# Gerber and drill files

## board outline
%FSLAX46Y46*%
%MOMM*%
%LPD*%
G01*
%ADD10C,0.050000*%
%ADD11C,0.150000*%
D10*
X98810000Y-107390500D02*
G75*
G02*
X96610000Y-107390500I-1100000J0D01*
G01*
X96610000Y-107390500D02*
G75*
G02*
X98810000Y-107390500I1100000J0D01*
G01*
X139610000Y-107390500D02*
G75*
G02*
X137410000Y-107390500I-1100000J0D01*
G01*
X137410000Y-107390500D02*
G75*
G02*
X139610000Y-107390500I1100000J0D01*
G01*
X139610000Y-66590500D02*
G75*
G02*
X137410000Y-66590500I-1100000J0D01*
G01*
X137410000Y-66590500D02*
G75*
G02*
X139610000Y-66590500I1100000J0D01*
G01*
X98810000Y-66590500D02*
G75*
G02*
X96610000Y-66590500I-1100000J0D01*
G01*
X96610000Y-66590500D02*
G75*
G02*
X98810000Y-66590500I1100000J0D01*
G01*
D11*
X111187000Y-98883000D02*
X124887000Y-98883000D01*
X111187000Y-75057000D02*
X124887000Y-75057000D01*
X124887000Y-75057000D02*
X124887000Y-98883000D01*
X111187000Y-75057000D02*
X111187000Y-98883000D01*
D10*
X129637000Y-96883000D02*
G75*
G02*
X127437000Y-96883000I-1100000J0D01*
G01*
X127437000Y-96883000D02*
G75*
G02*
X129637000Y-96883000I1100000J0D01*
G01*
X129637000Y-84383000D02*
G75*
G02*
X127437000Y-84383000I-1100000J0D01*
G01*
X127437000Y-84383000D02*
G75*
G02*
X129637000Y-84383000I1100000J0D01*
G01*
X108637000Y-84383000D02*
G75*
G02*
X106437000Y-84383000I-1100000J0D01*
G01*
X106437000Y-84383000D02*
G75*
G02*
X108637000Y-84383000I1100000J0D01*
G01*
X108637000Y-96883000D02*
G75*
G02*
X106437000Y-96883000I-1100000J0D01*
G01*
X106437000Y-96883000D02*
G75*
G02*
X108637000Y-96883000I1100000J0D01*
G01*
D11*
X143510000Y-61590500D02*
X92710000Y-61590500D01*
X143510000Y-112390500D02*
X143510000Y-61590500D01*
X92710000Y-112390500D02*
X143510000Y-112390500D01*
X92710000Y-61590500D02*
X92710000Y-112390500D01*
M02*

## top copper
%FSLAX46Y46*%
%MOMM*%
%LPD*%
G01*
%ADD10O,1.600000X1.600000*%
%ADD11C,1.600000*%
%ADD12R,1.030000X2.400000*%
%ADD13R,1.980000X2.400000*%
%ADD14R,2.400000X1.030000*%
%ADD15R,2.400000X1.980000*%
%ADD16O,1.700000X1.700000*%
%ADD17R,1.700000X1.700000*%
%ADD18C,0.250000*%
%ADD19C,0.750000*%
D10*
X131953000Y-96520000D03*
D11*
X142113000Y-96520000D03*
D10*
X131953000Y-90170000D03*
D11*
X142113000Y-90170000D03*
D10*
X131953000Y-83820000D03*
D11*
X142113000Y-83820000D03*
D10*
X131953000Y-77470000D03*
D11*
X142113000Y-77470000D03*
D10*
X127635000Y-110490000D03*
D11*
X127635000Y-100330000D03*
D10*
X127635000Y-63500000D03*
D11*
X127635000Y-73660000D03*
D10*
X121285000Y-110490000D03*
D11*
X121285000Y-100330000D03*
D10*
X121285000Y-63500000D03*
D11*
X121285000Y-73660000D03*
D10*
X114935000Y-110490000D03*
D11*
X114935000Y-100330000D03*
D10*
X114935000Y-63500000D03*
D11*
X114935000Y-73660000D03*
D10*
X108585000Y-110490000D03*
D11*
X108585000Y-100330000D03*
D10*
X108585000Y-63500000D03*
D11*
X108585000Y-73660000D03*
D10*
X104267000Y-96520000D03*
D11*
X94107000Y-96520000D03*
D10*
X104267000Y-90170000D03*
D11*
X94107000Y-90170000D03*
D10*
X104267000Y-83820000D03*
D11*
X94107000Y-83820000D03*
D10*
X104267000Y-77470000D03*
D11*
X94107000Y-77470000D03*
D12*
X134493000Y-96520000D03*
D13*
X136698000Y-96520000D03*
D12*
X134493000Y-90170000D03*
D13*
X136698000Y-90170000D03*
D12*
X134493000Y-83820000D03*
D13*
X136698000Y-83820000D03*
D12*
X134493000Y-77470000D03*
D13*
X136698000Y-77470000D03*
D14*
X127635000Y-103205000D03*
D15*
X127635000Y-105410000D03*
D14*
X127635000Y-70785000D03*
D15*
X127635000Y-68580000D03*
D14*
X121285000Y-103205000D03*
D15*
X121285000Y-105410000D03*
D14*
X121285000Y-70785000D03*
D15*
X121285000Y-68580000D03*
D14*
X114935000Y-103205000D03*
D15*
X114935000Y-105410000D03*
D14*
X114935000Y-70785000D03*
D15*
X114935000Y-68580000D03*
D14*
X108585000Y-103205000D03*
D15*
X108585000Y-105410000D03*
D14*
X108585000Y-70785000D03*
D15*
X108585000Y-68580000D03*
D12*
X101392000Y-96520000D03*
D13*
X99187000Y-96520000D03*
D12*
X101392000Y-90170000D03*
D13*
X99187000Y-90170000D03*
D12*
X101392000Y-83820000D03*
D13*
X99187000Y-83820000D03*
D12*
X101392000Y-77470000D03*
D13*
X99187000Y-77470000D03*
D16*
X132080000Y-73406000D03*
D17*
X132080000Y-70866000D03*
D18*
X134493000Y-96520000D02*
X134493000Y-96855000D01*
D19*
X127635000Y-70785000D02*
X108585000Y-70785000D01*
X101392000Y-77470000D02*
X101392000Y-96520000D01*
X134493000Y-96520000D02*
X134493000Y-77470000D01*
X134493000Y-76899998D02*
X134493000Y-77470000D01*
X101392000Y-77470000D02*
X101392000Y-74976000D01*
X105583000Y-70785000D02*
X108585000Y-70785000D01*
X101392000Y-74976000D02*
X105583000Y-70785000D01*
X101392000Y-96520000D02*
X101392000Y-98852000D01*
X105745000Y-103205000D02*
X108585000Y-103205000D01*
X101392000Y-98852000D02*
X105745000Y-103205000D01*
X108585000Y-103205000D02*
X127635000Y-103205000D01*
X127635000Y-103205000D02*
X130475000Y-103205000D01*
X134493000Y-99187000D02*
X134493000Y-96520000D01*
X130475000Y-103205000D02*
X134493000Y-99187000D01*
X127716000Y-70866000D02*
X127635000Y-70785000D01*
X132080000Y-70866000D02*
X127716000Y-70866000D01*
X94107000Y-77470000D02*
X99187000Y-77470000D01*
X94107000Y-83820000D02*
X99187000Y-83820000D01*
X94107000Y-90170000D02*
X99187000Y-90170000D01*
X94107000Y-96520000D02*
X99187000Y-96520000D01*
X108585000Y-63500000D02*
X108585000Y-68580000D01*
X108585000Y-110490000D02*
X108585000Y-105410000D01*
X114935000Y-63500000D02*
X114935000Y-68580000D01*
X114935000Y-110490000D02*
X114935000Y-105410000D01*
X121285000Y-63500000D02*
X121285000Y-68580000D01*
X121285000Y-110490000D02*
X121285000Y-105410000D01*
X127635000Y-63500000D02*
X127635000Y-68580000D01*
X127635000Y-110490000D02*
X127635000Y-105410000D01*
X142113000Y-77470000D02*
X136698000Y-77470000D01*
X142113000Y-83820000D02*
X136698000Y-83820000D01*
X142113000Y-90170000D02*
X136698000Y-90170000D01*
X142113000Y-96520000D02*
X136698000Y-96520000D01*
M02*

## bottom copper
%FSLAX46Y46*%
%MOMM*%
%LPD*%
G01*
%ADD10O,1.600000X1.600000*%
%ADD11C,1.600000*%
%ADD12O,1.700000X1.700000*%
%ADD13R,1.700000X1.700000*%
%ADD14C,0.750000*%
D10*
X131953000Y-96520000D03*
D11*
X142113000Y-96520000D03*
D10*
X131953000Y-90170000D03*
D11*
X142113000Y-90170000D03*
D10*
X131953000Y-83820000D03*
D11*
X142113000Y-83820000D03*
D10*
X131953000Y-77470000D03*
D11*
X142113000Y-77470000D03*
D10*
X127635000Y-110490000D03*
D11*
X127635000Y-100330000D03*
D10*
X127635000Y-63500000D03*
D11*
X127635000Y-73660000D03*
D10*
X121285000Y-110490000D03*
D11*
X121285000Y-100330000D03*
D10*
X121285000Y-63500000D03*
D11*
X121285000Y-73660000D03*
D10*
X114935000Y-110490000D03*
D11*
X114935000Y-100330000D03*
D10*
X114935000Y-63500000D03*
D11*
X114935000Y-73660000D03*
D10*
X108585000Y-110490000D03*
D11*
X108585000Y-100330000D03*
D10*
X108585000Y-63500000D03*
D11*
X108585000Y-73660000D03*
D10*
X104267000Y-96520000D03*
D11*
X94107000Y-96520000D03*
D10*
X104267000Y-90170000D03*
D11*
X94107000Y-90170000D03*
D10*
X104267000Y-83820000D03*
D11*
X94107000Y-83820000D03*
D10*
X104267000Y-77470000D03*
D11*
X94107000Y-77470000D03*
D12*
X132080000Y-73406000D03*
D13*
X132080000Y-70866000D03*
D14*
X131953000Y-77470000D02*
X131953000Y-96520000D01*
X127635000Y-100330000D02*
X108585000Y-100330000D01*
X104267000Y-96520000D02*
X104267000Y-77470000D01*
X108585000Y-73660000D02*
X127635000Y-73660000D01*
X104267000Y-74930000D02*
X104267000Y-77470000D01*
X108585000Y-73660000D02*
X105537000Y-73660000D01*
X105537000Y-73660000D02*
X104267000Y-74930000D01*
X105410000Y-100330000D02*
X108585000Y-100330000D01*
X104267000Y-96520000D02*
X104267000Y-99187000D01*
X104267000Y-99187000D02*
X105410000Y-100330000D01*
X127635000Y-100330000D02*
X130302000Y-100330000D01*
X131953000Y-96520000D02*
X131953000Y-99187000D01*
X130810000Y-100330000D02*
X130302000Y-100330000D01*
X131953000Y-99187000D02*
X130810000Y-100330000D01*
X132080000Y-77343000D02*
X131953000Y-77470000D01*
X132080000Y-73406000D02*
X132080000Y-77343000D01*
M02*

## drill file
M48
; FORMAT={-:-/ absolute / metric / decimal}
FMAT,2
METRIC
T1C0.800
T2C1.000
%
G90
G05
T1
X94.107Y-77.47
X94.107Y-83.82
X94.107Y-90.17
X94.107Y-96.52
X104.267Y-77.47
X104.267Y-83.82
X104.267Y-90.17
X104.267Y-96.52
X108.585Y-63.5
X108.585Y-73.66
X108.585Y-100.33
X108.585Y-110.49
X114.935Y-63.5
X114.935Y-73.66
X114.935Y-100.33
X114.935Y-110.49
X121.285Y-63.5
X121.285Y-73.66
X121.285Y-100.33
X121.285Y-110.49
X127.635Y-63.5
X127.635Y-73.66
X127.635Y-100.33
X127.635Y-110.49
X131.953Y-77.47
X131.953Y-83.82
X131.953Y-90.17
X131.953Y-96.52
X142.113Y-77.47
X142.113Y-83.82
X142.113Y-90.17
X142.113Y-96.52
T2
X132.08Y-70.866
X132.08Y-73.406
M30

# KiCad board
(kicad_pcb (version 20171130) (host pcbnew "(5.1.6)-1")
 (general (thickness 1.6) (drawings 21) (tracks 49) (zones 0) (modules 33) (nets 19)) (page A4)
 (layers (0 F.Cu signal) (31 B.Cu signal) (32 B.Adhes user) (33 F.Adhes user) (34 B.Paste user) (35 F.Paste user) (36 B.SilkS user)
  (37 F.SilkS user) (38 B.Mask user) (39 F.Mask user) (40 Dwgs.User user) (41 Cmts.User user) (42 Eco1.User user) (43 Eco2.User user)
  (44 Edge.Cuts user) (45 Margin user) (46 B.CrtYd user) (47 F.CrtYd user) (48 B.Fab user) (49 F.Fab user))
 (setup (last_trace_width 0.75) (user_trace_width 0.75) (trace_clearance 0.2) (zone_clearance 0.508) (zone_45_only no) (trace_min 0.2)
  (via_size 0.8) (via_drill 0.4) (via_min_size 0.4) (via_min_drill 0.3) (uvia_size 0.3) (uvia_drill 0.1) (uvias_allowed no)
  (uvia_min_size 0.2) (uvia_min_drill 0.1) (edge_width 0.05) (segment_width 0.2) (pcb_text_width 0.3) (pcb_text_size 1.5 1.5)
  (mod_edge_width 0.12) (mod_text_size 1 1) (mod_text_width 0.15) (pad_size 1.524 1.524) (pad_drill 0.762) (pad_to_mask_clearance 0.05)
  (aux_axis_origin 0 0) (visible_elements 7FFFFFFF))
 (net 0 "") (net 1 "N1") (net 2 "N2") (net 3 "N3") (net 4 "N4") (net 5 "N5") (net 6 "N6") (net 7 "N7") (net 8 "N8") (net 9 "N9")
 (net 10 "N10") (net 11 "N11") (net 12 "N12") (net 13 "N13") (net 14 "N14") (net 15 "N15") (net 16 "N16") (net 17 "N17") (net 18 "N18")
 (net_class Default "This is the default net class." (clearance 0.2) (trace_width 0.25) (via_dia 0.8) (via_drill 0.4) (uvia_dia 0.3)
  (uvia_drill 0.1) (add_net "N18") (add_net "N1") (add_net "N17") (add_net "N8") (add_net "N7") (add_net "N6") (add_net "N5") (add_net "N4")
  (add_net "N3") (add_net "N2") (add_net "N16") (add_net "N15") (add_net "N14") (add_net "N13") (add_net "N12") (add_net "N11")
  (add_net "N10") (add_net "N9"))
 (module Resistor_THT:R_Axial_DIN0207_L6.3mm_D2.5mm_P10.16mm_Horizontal (layer B.Cu) (at 142.113 96.52 180)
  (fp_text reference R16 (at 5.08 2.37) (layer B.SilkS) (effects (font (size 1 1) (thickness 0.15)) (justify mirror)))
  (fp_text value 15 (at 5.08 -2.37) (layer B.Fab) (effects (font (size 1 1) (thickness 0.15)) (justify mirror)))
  (pad 2 thru_hole oval (at 10.16 0 180) (size 1.6 1.6) (drill 0.8) (layers *.Cu *.Mask) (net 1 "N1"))
  (pad 1 thru_hole circle (at 0 0 180) (size 1.6 1.6) (drill 0.8) (layers *.Cu *.Mask) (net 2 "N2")))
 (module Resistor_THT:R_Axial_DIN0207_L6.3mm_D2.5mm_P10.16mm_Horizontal (layer B.Cu) (at 142.113 90.17 180)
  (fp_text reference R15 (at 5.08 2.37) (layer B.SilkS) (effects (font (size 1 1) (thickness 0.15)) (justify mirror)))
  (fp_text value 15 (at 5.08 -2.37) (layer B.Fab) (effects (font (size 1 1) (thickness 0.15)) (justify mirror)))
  (pad 2 thru_hole oval (at 10.16 0 180) (size 1.6 1.6) (drill 0.8) (layers *.Cu *.Mask) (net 1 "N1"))
  (pad 1 thru_hole circle (at 0 0 180) (size 1.6 1.6) (drill 0.8) (layers *.Cu *.Mask) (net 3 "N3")))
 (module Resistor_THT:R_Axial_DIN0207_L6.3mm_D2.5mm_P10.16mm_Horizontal (layer B.Cu) (at 142.113 83.82 180)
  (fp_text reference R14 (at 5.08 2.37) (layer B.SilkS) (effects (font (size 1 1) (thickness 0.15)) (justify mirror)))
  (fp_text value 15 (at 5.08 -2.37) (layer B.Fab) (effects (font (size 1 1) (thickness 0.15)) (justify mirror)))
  (pad 2 thru_hole oval (at 10.16 0 180) (size 1.6 1.6) (drill 0.8) (layers *.Cu *.Mask) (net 1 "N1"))
  (pad 1 thru_hole circle (at 0 0 180) (size 1.6 1.6) (drill 0.8) (layers *.Cu *.Mask) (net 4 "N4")))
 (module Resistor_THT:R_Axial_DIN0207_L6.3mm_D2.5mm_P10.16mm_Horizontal (layer B.Cu) (at 142.113 77.47 180)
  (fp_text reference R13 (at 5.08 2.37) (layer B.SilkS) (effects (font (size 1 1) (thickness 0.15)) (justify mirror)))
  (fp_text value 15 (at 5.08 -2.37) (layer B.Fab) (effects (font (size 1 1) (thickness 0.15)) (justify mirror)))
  (pad 2 thru_hole oval (at 10.16 0 180) (size 1.6 1.6) (drill 0.8) (layers *.Cu *.Mask) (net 1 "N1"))
  (pad 1 thru_hole circle (at 0 0 180) (size 1.6 1.6) (drill 0.8) (layers *.Cu *.Mask) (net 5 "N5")))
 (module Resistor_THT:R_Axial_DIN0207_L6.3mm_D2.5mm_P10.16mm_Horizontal (layer B.Cu) (at 127.635 100.33 270)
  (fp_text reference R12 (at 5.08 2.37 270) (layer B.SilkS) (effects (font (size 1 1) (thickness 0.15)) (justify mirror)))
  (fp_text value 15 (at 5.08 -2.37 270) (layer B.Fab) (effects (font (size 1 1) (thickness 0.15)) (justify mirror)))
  (pad 2 thru_hole oval (at 10.16 0 270) (size 1.6 1.6) (drill 0.8) (layers *.Cu *.Mask) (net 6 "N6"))
  (pad 1 thru_hole circle (at 0 0 270) (size 1.6 1.6) (drill 0.8) (layers *.Cu *.Mask) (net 1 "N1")))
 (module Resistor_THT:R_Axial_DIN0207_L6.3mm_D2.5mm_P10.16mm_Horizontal (layer B.Cu) (at 127.635 73.66 90)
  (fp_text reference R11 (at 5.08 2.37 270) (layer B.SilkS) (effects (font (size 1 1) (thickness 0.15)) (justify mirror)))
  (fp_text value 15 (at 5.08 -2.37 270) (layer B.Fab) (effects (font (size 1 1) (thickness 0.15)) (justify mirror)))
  (pad 2 thru_hole oval (at 10.16 0 90) (size 1.6 1.6) (drill 0.8) (layers *.Cu *.Mask) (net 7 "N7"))
  (pad 1 thru_hole circle (at 0 0 90) (size 1.6 1.6) (drill 0.8) (layers *.Cu *.Mask) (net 1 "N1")))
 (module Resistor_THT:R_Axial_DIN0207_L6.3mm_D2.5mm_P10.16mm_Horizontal (layer B.Cu) (at 121.285 100.33 270)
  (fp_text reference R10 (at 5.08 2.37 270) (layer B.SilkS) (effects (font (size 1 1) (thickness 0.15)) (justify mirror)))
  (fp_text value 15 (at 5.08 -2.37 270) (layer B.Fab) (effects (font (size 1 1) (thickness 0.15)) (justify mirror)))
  (pad 2 thru_hole oval (at 10.16 0 270) (size 1.6 1.6) (drill 0.8) (layers *.Cu *.Mask) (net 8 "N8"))
  (pad 1 thru_hole circle (at 0 0 270) (size 1.6 1.6) (drill 0.8) (layers *.Cu *.Mask) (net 1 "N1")))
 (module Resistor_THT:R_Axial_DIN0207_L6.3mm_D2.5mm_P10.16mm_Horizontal (layer B.Cu) (at 121.285 73.66 90)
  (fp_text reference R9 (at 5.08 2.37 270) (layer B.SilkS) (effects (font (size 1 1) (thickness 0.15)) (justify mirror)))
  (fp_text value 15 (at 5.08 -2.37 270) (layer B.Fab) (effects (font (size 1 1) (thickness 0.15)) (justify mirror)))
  (pad 2 thru_hole oval (at 10.16 0 90) (size 1.6 1.6) (drill 0.8) (layers *.Cu *.Mask) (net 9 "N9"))
  (pad 1 thru_hole circle (at 0 0 90) (size 1.6 1.6) (drill 0.8) (layers *.Cu *.Mask) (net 1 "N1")))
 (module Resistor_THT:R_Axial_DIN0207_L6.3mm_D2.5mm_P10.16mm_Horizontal (layer B.Cu) (at 114.935 100.33 270)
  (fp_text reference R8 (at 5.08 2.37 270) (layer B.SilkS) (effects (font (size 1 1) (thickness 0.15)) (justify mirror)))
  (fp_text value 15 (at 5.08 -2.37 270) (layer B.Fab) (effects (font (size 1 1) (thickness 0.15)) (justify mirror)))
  (pad 2 thru_hole oval (at 10.16 0 270) (size 1.6 1.6) (drill 0.8) (layers *.Cu *.Mask) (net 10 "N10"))
  (pad 1 thru_hole circle (at 0 0 270) (size 1.6 1.6) (drill 0.8) (layers *.Cu *.Mask) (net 1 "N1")))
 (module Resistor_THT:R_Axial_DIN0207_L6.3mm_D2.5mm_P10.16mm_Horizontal (layer B.Cu) (at 114.935 73.66 90)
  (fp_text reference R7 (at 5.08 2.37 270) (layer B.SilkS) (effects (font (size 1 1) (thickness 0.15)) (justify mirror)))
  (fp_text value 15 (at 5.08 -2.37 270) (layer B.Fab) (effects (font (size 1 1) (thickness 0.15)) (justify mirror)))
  (pad 2 thru_hole oval (at 10.16 0 90) (size 1.6 1.6) (drill 0.8) (layers *.Cu *.Mask) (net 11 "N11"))
  (pad 1 thru_hole circle (at 0 0 90) (size 1.6 1.6) (drill 0.8) (layers *.Cu *.Mask) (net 1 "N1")))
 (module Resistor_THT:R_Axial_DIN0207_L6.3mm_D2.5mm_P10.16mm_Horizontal (layer B.Cu) (at 108.585 100.33 270)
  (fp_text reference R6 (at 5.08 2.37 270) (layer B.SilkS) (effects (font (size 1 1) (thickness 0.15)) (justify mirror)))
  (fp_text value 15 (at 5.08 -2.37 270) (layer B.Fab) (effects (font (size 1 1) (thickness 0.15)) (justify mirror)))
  (pad 2 thru_hole oval (at 10.16 0 270) (size 1.6 1.6) (drill 0.8) (layers *.Cu *.Mask) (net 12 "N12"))
  (pad 1 thru_hole circle (at 0 0 270) (size 1.6 1.6) (drill 0.8) (layers *.Cu *.Mask) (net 1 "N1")))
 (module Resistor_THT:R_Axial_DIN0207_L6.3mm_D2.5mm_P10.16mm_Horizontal (layer B.Cu) (at 108.585 73.66 90)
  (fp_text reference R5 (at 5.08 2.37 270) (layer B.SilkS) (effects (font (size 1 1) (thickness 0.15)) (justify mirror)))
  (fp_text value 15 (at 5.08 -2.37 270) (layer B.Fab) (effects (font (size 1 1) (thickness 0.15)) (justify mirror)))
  (pad 2 thru_hole oval (at 10.16 0 90) (size 1.6 1.6) (drill 0.8) (layers *.Cu *.Mask) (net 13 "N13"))
  (pad 1 thru_hole circle (at 0 0 90) (size 1.6 1.6) (drill 0.8) (layers *.Cu *.Mask) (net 1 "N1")))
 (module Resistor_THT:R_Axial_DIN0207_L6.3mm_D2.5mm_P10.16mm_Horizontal (layer B.Cu) (at 94.107 96.52)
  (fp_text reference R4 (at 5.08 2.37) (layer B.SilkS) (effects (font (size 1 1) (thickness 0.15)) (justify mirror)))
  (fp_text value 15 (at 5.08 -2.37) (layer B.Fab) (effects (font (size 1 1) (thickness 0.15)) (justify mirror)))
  (pad 2 thru_hole oval (at 10.16 0) (size 1.6 1.6) (drill 0.8) (layers *.Cu *.Mask) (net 1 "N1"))
  (pad 1 thru_hole circle (at 0 0) (size 1.6 1.6) (drill 0.8) (layers *.Cu *.Mask) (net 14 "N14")))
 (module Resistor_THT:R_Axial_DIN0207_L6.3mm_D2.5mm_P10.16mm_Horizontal (layer B.Cu) (at 94.107 90.17)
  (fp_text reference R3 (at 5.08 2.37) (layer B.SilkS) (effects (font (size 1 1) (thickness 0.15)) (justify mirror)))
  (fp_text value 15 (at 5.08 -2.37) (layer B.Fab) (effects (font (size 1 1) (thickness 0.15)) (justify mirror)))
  (pad 2 thru_hole oval (at 10.16 0) (size 1.6 1.6) (drill 0.8) (layers *.Cu *.Mask) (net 1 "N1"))
  (pad 1 thru_hole circle (at 0 0) (size 1.6 1.6) (drill 0.8) (layers *.Cu *.Mask) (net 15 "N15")))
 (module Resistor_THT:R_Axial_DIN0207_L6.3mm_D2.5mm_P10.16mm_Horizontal (layer B.Cu) (at 94.107 83.82)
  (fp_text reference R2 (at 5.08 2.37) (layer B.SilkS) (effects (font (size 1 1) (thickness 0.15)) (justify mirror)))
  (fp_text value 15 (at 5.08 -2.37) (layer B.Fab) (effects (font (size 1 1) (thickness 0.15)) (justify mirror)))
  (pad 2 thru_hole oval (at 10.16 0) (size 1.6 1.6) (drill 0.8) (layers *.Cu *.Mask) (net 1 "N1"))
  (pad 1 thru_hole circle (at 0 0) (size 1.6 1.6) (drill 0.8) (layers *.Cu *.Mask) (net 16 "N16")))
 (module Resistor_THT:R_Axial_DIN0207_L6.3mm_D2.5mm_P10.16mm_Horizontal (layer B.Cu) (at 94.107 77.47)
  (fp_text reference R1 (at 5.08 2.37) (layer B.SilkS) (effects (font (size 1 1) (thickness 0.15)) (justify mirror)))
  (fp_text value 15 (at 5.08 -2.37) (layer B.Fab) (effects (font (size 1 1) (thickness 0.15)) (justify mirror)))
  (pad 2 thru_hole oval (at 10.16 0) (size 1.6 1.6) (drill 0.8) (layers *.Cu *.Mask) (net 1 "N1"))
  (pad 1 thru_hole circle (at 0 0) (size 1.6 1.6) (drill 0.8) (layers *.Cu *.Mask) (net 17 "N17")))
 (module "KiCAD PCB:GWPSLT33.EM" (layer F.Cu) (at 135.838 96.52 180)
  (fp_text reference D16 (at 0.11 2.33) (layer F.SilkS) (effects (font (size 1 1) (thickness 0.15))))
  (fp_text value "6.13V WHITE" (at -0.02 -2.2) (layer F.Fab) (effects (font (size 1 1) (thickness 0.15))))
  (pad 2 smd rect (at 1.345 0 180) (size 1.03 2.4) (layers F.Cu F.Paste F.Mask) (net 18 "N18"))
  (pad 1 smd rect (at -0.86 0 180) (size 1.98 2.4) (layers F.Cu F.Paste F.Mask) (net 2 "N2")))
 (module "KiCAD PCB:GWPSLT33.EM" (layer F.Cu) (at 135.838 90.17 180)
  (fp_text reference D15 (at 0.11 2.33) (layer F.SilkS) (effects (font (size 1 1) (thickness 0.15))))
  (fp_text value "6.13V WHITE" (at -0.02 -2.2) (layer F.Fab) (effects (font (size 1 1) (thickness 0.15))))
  (pad 2 smd rect (at 1.345 0 180) (size 1.03 2.4) (layers F.Cu F.Paste F.Mask) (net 18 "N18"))
  (pad 1 smd rect (at -0.86 0 180) (size 1.98 2.4) (layers F.Cu F.Paste F.Mask) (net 3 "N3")))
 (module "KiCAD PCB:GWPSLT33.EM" (layer F.Cu) (at 135.838 83.82 180)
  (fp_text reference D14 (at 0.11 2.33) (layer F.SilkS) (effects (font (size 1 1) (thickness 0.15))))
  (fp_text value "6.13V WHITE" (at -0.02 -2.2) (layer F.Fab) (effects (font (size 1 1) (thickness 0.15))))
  (pad 2 smd rect (at 1.345 0 180) (size 1.03 2.4) (layers F.Cu F.Paste F.Mask) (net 18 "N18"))
  (pad 1 smd rect (at -0.86 0 180) (size 1.98 2.4) (layers F.Cu F.Paste F.Mask) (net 4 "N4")))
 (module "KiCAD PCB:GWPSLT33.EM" (layer F.Cu) (at 135.838 77.47 180)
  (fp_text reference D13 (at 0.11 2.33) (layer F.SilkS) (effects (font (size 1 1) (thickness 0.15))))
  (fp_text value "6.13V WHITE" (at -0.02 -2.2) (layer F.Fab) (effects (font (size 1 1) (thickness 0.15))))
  (pad 2 smd rect (at 1.345 0 180) (size 1.03 2.4) (layers F.Cu F.Paste F.Mask) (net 18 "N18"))
  (pad 1 smd rect (at -0.86 0 180) (size 1.98 2.4) (layers F.Cu F.Paste F.Mask) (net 5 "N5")))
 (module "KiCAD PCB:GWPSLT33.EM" (layer F.Cu) (at 127.635 104.55 90)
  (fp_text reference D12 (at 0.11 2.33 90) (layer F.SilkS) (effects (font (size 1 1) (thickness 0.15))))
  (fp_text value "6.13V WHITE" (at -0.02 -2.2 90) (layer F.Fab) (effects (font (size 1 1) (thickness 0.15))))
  (pad 2 smd rect (at 1.345 0 90) (size 1.03 2.4) (layers F.Cu F.Paste F.Mask) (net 18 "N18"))
  (pad 1 smd rect (at -0.86 0 90) (size 1.98 2.4) (layers F.Cu F.Paste F.Mask) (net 6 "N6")))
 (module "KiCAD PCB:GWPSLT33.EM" (layer F.Cu) (at 127.635 69.44 270)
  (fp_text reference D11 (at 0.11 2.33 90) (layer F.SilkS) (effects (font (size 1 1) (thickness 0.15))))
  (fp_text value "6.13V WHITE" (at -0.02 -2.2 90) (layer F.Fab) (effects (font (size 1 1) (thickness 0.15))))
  (pad 2 smd rect (at 1.345 0 270) (size 1.03 2.4) (layers F.Cu F.Paste F.Mask) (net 18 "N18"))
  (pad 1 smd rect (at -0.86 0 270) (size 1.98 2.4) (layers F.Cu F.Paste F.Mask) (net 7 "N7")))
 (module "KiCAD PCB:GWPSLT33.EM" (layer F.Cu) (at 121.285 104.55 90)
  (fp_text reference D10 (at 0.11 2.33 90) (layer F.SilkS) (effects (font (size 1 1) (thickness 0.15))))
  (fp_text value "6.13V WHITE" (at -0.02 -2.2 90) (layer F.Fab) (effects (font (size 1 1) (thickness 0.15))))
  (pad 2 smd rect (at 1.345 0 90) (size 1.03 2.4) (layers F.Cu F.Paste F.Mask) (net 18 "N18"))
  (pad 1 smd rect (at -0.86 0 90) (size 1.98 2.4) (layers F.Cu F.Paste F.Mask) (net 8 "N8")))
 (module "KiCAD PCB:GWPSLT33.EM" (layer F.Cu) (at 121.285 69.44 270)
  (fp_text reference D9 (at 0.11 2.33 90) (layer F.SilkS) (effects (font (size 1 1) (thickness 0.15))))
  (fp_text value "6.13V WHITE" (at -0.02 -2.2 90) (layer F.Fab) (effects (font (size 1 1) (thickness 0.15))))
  (pad 2 smd rect (at 1.345 0 270) (size 1.03 2.4) (layers F.Cu F.Paste F.Mask) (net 18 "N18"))
  (pad 1 smd rect (at -0.86 0 270) (size 1.98 2.4) (layers F.Cu F.Paste F.Mask) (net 9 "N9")))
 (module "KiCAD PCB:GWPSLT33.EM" (layer F.Cu) (at 114.935 104.55 90)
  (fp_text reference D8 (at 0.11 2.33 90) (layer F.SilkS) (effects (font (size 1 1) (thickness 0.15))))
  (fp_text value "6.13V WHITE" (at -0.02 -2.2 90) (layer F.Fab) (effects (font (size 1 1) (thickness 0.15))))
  (pad 2 smd rect (at 1.345 0 90) (size 1.03 2.4) (layers F.Cu F.Paste F.Mask) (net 18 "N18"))
  (pad 1 smd rect (at -0.86 0 90) (size 1.98 2.4) (layers F.Cu F.Paste F.Mask) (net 10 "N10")))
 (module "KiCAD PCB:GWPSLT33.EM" (layer F.Cu) (at 114.935 69.44 270)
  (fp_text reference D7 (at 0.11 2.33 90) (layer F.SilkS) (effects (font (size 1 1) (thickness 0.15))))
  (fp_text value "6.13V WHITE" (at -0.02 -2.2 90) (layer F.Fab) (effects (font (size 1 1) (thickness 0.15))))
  (pad 2 smd rect (at 1.345 0 270) (size 1.03 2.4) (layers F.Cu F.Paste F.Mask) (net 18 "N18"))
  (pad 1 smd rect (at -0.86 0 270) (size 1.98 2.4) (layers F.Cu F.Paste F.Mask) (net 11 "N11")))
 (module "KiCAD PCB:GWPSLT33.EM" (layer F.Cu) (at 108.585 104.55 90)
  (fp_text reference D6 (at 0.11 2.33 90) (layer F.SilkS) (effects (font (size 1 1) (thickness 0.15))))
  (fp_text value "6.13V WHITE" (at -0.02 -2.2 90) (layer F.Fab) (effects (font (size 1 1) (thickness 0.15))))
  (pad 2 smd rect (at 1.345 0 90) (size 1.03 2.4) (layers F.Cu F.Paste F.Mask) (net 18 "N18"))
  (pad 1 smd rect (at -0.86 0 90) (size 1.98 2.4) (layers F.Cu F.Paste F.Mask) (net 12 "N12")))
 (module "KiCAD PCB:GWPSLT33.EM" (layer F.Cu) (at 108.585 69.44 270)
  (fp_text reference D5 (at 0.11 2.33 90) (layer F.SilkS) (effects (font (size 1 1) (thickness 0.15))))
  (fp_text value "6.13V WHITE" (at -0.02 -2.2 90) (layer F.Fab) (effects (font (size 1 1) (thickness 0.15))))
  (pad 2 smd rect (at 1.345 0 270) (size 1.03 2.4) (layers F.Cu F.Paste F.Mask) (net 18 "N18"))
  (pad 1 smd rect (at -0.86 0 270) (size 1.98 2.4) (layers F.Cu F.Paste F.Mask) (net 13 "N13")))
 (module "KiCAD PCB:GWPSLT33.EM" (layer F.Cu) (at 100.047 96.52)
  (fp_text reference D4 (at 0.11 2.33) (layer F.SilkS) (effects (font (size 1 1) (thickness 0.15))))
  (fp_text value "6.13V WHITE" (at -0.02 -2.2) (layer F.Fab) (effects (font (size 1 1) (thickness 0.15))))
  (pad 2 smd rect (at 1.345 0) (size 1.03 2.4) (layers F.Cu F.Paste F.Mask) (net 18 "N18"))
  (pad 1 smd rect (at -0.86 0) (size 1.98 2.4) (layers F.Cu F.Paste F.Mask) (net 14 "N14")))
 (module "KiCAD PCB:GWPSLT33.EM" (layer F.Cu) (at 100.047 90.17)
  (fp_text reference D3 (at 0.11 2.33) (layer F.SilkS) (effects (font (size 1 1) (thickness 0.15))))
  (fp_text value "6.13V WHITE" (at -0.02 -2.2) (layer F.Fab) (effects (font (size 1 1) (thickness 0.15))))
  (pad 2 smd rect (at 1.345 0) (size 1.03 2.4) (layers F.Cu F.Paste F.Mask) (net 18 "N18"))
  (pad 1 smd rect (at -0.86 0) (size 1.98 2.4) (layers F.Cu F.Paste F.Mask) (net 15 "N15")))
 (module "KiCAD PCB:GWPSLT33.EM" (layer F.Cu) (at 100.047 83.82)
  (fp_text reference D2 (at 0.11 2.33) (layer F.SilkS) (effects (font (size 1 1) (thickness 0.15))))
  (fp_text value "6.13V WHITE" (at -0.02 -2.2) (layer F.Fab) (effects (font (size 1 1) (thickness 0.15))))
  (pad 2 smd rect (at 1.345 0) (size 1.03 2.4) (layers F.Cu F.Paste F.Mask) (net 18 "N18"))
  (pad 1 smd rect (at -0.86 0) (size 1.98 2.4) (layers F.Cu F.Paste F.Mask) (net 16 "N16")))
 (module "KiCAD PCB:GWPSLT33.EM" (layer F.Cu) (at 100.047 77.47)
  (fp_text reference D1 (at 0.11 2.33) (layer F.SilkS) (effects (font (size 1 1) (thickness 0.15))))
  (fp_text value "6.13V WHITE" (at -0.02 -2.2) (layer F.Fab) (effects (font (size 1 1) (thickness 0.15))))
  (pad 2 smd rect (at 1.345 0) (size 1.03 2.4) (layers F.Cu F.Paste F.Mask) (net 18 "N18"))
  (pad 1 smd rect (at -0.86 0) (size 1.98 2.4) (layers F.Cu F.Paste F.Mask) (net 17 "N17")))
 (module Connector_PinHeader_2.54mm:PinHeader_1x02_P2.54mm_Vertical (layer F.Cu) (at 132.08 70.866)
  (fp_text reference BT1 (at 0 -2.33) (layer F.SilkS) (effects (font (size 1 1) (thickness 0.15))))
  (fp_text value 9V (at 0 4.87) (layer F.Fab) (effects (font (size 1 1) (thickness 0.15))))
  (pad 2 thru_hole oval (at 0 2.54) (size 1.7 1.7) (drill 1) (layers *.Cu *.Mask) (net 1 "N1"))
  (pad 1 thru_hole rect (at 0 0) (size 1.7 1.7) (drill 1) (layers *.Cu *.Mask) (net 18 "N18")))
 (gr_circle (center 97.71 107.3905) (end 98.81 107.3905) (layer Edge.Cuts) (width 0.05))
 (gr_circle (center 138.51 107.3905) (end 139.61 107.3905) (layer Edge.Cuts) (width 0.05))
 (gr_circle (center 138.51 66.5905) (end 139.61 66.5905) (layer Edge.Cuts) (width 0.05))
 (gr_circle (center 97.71 66.5905) (end 98.81 66.5905) (layer Edge.Cuts) (width 0.05))
 (gr_line (start 111.187 98.883) (end 124.887 98.883) (layer Edge.Cuts) (width 0.15))
 (gr_line (start 111.187 75.057) (end 124.887 75.057) (layer Edge.Cuts) (width 0.15))
 (gr_line (start 124.887 75.057) (end 124.887 98.883) (layer Edge.Cuts) (width 0.15))
 (gr_line (start 111.187 75.057) (end 111.187 98.883) (layer Edge.Cuts) (width 0.15))
 (gr_circle (center 128.537 96.883) (end 129.637 96.883) (layer Edge.Cuts) (width 0.05))
 (gr_circle (center 128.537 84.383) (end 129.637 84.383) (layer Edge.Cuts) (width 0.05))
 (gr_circle (center 107.537 84.383) (end 108.637 84.383) (layer Edge.Cuts) (width 0.05))
 (gr_circle (center 107.537 96.883) (end 108.637 96.883) (layer Edge.Cuts) (width 0.05))
 (gr_line (start 143.51 61.5905) (end 92.71 61.5905) (layer Edge.Cuts) (width 0.15))
 (gr_line (start 143.51 112.3905) (end 143.51 61.5905) (layer Edge.Cuts) (width 0.15))
 (gr_line (start 92.71 112.3905) (end 143.51 112.3905) (layer Edge.Cuts) (width 0.15))
 (gr_line (start 92.71 61.5905) (end 92.71 112.3905) (layer Edge.Cuts) (width 0.15))
 (segment (start 131.953 77.47) (end 131.953 96.52) (width 0.75) (layer B.Cu) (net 1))
 (segment (start 127.635 100.33) (end 108.585 100.33) (width 0.75) (layer B.Cu) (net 1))
 (segment (start 104.267 96.52) (end 104.267 77.47) (width 0.75) (layer B.Cu) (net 1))
 (segment (start 108.585 73.66) (end 127.635 73.66) (width 0.75) (layer B.Cu) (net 1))
 (segment (start 104.267 74.93) (end 104.267 77.47) (width 0.75) (layer B.Cu) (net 1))
 (segment (start 108.585 73.66) (end 105.537 73.66) (width 0.75) (layer B.Cu) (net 1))
 (segment (start 105.537 73.66) (end 104.267 74.93) (width 0.75) (layer B.Cu) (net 1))
 (segment (start 105.41 100.33) (end 108.585 100.33) (width 0.75) (layer B.Cu) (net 1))
 (segment (start 104.267 96.52) (end 104.267 99.187) (width 0.75) (layer B.Cu) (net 1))
 (segment (start 104.267 99.187) (end 105.41 100.33) (width 0.75) (layer B.Cu) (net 1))
 (segment (start 127.635 100.33) (end 130.302 100.33) (width 0.75) (layer B.Cu) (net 1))
 (segment (start 131.953 96.52) (end 131.953 99.187) (width 0.75) (layer B.Cu) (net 1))
 (segment (start 130.81 100.33) (end 130.302 100.33) (width 0.75) (layer B.Cu) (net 1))
 (segment (start 131.953 99.187) (end 130.81 100.33) (width 0.75) (layer B.Cu) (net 1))
 (segment (start 132.08 77.343) (end 131.953 77.47) (width 0.75) (layer B.Cu) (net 1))
 (segment (start 132.08 73.406) (end 132.08 77.343) (width 0.75) (layer B.Cu) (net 1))
 (segment (start 134.493 96.52) (end 134.493 96.855) (width 0.25) (layer F.Cu) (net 18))
 (segment (start 127.635 70.785) (end 108.585 70.785) (width 0.75) (layer F.Cu) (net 18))
 (segment (start 101.392 77.47) (end 101.392 96.52) (width 0.75) (layer F.Cu) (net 18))
 (segment (start 134.493 96.52) (end 134.493 77.47) (width 0.75) (layer F.Cu) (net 18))
 (segment (start 134.493 76.899998) (end 134.493 77.47) (width 0.75) (layer F.Cu) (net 18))
 (segment (start 101.392 77.47) (end 101.392 74.976) (width 0.75) (layer F.Cu) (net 18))
 (segment (start 105.583 70.785) (end 108.585 70.785) (width 0.75) (layer F.Cu) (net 18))
 (segment (start 101.392 74.976) (end 105.583 70.785) (width 0.75) (layer F.Cu) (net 18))
 (segment (start 101.392 96.52) (end 101.392 98.852) (width 0.75) (layer F.Cu) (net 18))
 (segment (start 105.745 103.205) (end 108.585 103.205) (width 0.75) (layer F.Cu) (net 18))
 (segment (start 101.392 98.852) (end 105.745 103.205) (width 0.75) (layer F.Cu) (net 18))
 (segment (start 108.585 103.205) (end 127.635 103.205) (width 0.75) (layer F.Cu) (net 18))
 (segment (start 127.635 103.205) (end 130.475 103.205) (width 0.75) (layer F.Cu) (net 18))
 (segment (start 134.493 99.187) (end 134.493 96.52) (width 0.75) (layer F.Cu) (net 18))
 (segment (start 130.475 103.205) (end 134.493 99.187) (width 0.75) (layer F.Cu) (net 18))
 (segment (start 127.716 70.866) (end 127.635 70.785) (width 0.75) (layer F.Cu) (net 18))
 (segment (start 132.08 70.866) (end 127.716 70.866) (width 0.75) (layer F.Cu) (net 18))
 (segment (start 94.107 77.47) (end 99.187 77.47) (width 0.75) (layer F.Cu) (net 17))
 (segment (start 94.107 83.82) (end 99.187 83.82) (width 0.75) (layer F.Cu) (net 16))
 (segment (start 94.107 90.17) (end 99.187 90.17) (width 0.75) (layer F.Cu) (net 15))
 (segment (start 94.107 96.52) (end 99.187 96.52) (width 0.75) (layer F.Cu) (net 14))
 (segment (start 108.585 63.5) (end 108.585 68.58) (width 0.75) (layer F.Cu) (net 13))
 (segment (start 108.585 110.49) (end 108.585 105.41) (width 0.75) (layer F.Cu) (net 12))
 (segment (start 114.935 63.5) (end 114.935 68.58) (width 0.75) (layer F.Cu) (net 11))
 (segment (start 114.935 110.49) (end 114.935 105.41) (width 0.75) (layer F.Cu) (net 10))
 (segment (start 121.285 63.5) (end 121.285 68.58) (width 0.75) (layer F.Cu) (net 9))
 (segment (start 121.285 110.49) (end 121.285 105.41) (width 0.75) (layer F.Cu) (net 8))
 (segment (start 127.635 63.5) (end 127.635 68.58) (width 0.75) (layer F.Cu) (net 7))
 (segment (start 127.635 110.49) (end 127.635 105.41) (width 0.75) (layer F.Cu) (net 6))
 (segment (start 142.113 77.47) (end 136.698 77.47) (width 0.75) (layer F.Cu) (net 5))
 (segment (start 142.113 83.82) (end 136.698 83.82) (width 0.75) (layer F.Cu) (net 4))
 (segment (start 142.113 90.17) (end 136.698 90.17) (width 0.75) (layer F.Cu) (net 3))
 (segment (start 142.113 96.52) (end 136.698 96.52) (width 0.75) (layer F.Cu) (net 2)))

